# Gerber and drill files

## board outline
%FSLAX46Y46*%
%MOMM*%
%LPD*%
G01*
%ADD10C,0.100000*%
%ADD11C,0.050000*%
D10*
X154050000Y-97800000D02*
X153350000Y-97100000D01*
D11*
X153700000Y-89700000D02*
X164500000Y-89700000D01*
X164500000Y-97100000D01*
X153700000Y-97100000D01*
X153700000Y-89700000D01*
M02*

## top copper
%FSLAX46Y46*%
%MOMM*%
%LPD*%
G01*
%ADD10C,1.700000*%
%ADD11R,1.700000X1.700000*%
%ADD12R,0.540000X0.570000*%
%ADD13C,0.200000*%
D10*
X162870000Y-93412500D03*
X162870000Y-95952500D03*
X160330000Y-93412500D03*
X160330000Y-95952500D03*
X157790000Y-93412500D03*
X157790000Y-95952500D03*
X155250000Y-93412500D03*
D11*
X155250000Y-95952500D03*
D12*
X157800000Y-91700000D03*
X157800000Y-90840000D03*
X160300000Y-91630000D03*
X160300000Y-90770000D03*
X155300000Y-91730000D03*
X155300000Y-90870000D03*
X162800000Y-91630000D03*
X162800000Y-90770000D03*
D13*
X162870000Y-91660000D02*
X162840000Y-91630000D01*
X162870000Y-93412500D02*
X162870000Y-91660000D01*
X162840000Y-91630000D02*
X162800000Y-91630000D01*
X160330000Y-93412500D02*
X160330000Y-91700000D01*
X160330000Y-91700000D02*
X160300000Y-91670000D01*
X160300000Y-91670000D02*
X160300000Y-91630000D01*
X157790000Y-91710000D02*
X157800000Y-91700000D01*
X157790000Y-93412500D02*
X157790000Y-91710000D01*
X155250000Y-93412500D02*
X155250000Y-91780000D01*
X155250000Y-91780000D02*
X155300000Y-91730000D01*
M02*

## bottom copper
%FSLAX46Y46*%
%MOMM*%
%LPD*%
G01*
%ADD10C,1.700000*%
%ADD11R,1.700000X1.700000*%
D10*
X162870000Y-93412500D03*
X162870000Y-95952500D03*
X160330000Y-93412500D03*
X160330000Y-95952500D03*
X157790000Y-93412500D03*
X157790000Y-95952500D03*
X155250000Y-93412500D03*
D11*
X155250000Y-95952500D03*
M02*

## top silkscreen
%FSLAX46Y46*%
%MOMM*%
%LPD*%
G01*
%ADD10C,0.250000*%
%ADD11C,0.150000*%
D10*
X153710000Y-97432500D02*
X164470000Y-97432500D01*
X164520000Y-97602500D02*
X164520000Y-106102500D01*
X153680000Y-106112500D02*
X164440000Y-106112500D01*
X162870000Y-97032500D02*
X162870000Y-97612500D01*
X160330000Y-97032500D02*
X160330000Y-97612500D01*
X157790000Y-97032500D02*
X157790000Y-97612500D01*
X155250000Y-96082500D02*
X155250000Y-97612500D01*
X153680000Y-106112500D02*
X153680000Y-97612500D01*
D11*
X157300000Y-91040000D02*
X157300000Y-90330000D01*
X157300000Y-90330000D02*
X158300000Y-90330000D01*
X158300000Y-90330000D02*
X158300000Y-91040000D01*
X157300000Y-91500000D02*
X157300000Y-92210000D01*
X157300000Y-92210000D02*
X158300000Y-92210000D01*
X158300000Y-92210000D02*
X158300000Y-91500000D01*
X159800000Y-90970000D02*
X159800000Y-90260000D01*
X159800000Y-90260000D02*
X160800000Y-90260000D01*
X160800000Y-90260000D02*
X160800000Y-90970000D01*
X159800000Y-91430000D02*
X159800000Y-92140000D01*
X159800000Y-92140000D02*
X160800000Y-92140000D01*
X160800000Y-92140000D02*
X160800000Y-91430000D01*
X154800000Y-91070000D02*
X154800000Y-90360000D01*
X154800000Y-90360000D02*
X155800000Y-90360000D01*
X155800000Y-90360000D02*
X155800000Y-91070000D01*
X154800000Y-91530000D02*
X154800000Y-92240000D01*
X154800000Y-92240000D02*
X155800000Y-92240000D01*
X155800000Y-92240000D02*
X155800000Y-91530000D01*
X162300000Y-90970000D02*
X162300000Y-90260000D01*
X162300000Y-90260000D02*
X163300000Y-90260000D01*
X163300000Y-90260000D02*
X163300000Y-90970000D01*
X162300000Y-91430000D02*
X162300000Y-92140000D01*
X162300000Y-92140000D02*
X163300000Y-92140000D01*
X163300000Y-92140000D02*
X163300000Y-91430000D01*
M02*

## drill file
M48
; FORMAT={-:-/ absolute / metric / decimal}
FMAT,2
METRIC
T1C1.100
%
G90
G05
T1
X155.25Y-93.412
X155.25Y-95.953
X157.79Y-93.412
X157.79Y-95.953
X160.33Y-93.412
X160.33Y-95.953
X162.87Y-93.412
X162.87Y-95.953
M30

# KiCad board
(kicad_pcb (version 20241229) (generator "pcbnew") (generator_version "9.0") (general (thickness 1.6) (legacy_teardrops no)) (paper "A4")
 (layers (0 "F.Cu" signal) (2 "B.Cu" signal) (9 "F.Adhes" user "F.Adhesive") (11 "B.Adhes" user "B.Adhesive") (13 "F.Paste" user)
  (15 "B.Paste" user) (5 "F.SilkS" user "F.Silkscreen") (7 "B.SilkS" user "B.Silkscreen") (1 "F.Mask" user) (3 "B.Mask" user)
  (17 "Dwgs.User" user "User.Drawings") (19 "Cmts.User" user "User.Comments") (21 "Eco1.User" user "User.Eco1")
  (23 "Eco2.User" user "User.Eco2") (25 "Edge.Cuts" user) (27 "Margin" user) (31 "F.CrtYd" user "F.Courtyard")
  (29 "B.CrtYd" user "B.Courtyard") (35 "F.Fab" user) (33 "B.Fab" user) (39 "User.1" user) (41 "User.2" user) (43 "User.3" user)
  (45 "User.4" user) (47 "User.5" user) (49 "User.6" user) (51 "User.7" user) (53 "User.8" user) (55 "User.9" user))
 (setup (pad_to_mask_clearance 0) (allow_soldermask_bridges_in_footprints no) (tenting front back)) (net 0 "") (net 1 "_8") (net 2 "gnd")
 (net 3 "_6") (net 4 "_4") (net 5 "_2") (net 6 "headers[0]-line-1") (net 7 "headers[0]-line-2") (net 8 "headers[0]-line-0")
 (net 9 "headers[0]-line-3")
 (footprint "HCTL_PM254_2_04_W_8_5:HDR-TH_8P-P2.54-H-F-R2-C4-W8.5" (layer "F.Cu") (at 159.06 94.6825 0)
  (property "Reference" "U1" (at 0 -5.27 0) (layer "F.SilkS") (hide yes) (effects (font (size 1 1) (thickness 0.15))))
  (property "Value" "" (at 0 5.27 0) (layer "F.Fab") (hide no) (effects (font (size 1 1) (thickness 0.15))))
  (fp_line (start -5.35 2.75) (end 5.41 2.75) (stroke (width 0.25) (type solid)) (layer "F.SilkS"))
  (fp_line (start 5.46 2.92) (end 5.46 11.42) (stroke (width 0.25) (type solid)) (layer "F.SilkS"))
  (fp_line (start -5.38 11.43) (end 5.38 11.43) (stroke (width 0.25) (type solid)) (layer "F.SilkS"))
  (fp_line (start 3.81 2.35) (end 3.81 2.93) (stroke (width 0.25) (type solid)) (layer "F.SilkS"))
  (fp_line (start 1.27 2.35) (end 1.27 2.93) (stroke (width 0.25) (type solid)) (layer "F.SilkS"))
  (fp_line (start -1.27 2.35) (end -1.27 2.93) (stroke (width 0.25) (type solid)) (layer "F.SilkS"))
  (fp_line (start -3.81 1.4) (end -3.81 2.93) (stroke (width 0.25) (type solid)) (layer "F.SilkS"))
  (fp_line (start -5.38 11.43) (end -5.38 2.93) (stroke (width 0.25) (type solid)) (layer "F.SilkS"))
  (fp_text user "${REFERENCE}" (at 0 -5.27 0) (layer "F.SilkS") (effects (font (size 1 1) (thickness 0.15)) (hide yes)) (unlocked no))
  (pad "8" thru_hole circle (at 3.81 -1.27 0) (size 1.7 1.7) (drill 1.1000231999999999) (layers "*.Cu" "*.Mask") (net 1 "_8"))
  (pad "7" thru_hole circle (at 3.81 1.27 0) (size 1.7 1.7) (drill 1.1000231999999999) (layers "*.Cu" "*.Mask") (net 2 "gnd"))
  (pad "6" thru_hole circle (at 1.27 -1.27 0) (size 1.7 1.7) (drill 1.1000231999999999) (layers "*.Cu" "*.Mask") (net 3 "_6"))
  (pad "5" thru_hole circle (at 1.27 1.27 0) (size 1.7 1.7) (drill 1.1000231999999999) (layers "*.Cu" "*.Mask") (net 2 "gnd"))
  (pad "4" thru_hole circle (at -1.27 -1.27 0) (size 1.7 1.7) (drill 1.1000231999999999) (layers "*.Cu" "*.Mask") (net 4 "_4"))
  (pad "3" thru_hole circle (at -1.27 1.27 0) (size 1.7 1.7) (drill 1.1000231999999999) (layers "*.Cu" "*.Mask") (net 2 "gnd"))
  (pad "2" thru_hole circle (at -3.81 -1.27 0) (size 1.7 1.7) (drill 1.1000231999999999) (layers "*.Cu" "*.Mask") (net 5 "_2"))
  (pad "1" thru_hole rect (at -3.81 1.27 0) (size 1.7 1.7) (drill 1.1000231999999999) (layers "*.Cu" "*.Mask") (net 2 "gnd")))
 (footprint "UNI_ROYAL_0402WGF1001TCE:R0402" (layer "F.Cu") (at 157.8 91.27 -90)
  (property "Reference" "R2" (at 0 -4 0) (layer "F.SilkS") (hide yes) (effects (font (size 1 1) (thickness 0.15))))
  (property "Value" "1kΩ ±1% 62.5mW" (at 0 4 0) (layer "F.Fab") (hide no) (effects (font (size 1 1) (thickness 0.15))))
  (fp_line (start -0.23 0.5) (end -0.94 0.5) (stroke (width 0.15) (type solid)) (layer "F.SilkS"))
  (fp_line (start -0.94 0.5) (end -0.94 -0.5) (stroke (width 0.15) (type solid)) (layer "F.SilkS"))
  (fp_line (start -0.94 -0.5) (end -0.23 -0.5) (stroke (width 0.15) (type solid)) (layer "F.SilkS"))
  (fp_line (start 0.23 0.5) (end 0.94 0.5) (stroke (width 0.15) (type solid)) (layer "F.SilkS"))
  (fp_line (start 0.94 0.5) (end 0.94 -0.5) (stroke (width 0.15) (type solid)) (layer "F.SilkS"))
  (fp_line (start 0.94 -0.5) (end 0.23 -0.5) (stroke (width 0.15) (type solid)) (layer "F.SilkS"))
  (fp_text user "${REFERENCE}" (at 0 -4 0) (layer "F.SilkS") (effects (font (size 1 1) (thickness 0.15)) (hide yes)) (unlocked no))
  (pad "2" smd rect (at 0.43 0 -90) (size 0.57 0.54) (layers "F.Cu" "F.Paste" "F.Mask") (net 4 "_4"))
  (pad "1" smd rect (at -0.43 0 -90) (size 0.57 0.54) (layers "F.Cu" "F.Paste" "F.Mask") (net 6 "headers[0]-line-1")))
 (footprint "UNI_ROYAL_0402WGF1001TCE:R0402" (layer "F.Cu") (at 160.3 91.2 -90)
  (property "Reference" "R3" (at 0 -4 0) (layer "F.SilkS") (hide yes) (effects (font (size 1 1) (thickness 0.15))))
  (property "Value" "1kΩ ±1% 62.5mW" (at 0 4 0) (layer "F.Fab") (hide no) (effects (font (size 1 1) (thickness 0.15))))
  (fp_line (start -0.23 0.5) (end -0.94 0.5) (stroke (width 0.15) (type solid)) (layer "F.SilkS"))
  (fp_line (start -0.94 0.5) (end -0.94 -0.5) (stroke (width 0.15) (type solid)) (layer "F.SilkS"))
  (fp_line (start -0.94 -0.5) (end -0.23 -0.5) (stroke (width 0.15) (type solid)) (layer "F.SilkS"))
  (fp_line (start 0.23 0.5) (end 0.94 0.5) (stroke (width 0.15) (type solid)) (layer "F.SilkS"))
  (fp_line (start 0.94 0.5) (end 0.94 -0.5) (stroke (width 0.15) (type solid)) (layer "F.SilkS"))
  (fp_line (start 0.94 -0.5) (end 0.23 -0.5) (stroke (width 0.15) (type solid)) (layer "F.SilkS"))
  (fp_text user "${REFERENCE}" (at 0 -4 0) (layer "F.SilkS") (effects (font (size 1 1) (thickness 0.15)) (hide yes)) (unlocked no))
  (pad "2" smd rect (at 0.43 0 -90) (size 0.57 0.54) (layers "F.Cu" "F.Paste" "F.Mask") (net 3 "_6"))
  (pad "1" smd rect (at -0.43 0 -90) (size 0.57 0.54) (layers "F.Cu" "F.Paste" "F.Mask") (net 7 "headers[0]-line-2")))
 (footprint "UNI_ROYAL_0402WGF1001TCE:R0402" (layer "F.Cu") (at 155.3 91.3 -90)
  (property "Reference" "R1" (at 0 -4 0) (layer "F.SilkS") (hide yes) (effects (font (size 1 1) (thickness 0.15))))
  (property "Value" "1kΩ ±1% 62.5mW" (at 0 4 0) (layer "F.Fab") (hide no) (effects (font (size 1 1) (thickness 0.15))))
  (fp_line (start -0.23 0.5) (end -0.94 0.5) (stroke (width 0.15) (type solid)) (layer "F.SilkS"))
  (fp_line (start -0.94 0.5) (end -0.94 -0.5) (stroke (width 0.15) (type solid)) (layer "F.SilkS"))
  (fp_line (start -0.94 -0.5) (end -0.23 -0.5) (stroke (width 0.15) (type solid)) (layer "F.SilkS"))
  (fp_line (start 0.23 0.5) (end 0.94 0.5) (stroke (width 0.15) (type solid)) (layer "F.SilkS"))
  (fp_line (start 0.94 0.5) (end 0.94 -0.5) (stroke (width 0.15) (type solid)) (layer "F.SilkS"))
  (fp_line (start 0.94 -0.5) (end 0.23 -0.5) (stroke (width 0.15) (type solid)) (layer "F.SilkS"))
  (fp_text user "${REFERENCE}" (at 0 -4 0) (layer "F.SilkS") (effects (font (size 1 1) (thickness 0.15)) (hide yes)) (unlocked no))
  (pad "2" smd rect (at 0.43 0 -90) (size 0.57 0.54) (layers "F.Cu" "F.Paste" "F.Mask") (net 5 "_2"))
  (pad "1" smd rect (at -0.43 0 -90) (size 0.57 0.54) (layers "F.Cu" "F.Paste" "F.Mask") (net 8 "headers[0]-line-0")))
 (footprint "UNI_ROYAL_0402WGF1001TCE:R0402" (layer "F.Cu") (at 162.8 91.2 -90)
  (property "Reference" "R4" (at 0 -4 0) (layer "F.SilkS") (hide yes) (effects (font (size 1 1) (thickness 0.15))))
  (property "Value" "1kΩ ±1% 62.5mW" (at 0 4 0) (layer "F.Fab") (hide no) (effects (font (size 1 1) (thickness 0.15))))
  (fp_line (start -0.23 0.5) (end -0.94 0.5) (stroke (width 0.15) (type solid)) (layer "F.SilkS"))
  (fp_line (start -0.94 0.5) (end -0.94 -0.5) (stroke (width 0.15) (type solid)) (layer "F.SilkS"))
  (fp_line (start -0.94 -0.5) (end -0.23 -0.5) (stroke (width 0.15) (type solid)) (layer "F.SilkS"))
  (fp_line (start 0.23 0.5) (end 0.94 0.5) (stroke (width 0.15) (type solid)) (layer "F.SilkS"))
  (fp_line (start 0.94 0.5) (end 0.94 -0.5) (stroke (width 0.15) (type solid)) (layer "F.SilkS"))
  (fp_line (start 0.94 -0.5) (end 0.23 -0.5) (stroke (width 0.15) (type solid)) (layer "F.SilkS"))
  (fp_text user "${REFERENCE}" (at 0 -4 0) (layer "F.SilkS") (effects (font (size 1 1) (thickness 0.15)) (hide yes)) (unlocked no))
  (pad "2" smd rect (at 0.43 0 -90) (size 0.57 0.54) (layers "F.Cu" "F.Paste" "F.Mask") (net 1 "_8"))
  (pad "1" smd rect (at -0.43 0 -90) (size 0.57 0.54) (layers "F.Cu" "F.Paste" "F.Mask") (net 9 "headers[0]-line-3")))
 (segment (start 162.87 91.66) (end 162.84 91.63) (width 0.2) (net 1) (layer "F.Cu"))
 (segment (start 162.87 93.4125) (end 162.87 91.66) (width 0.2) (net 1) (layer "F.Cu"))
 (segment (start 162.84 91.63) (end 162.8 91.63) (width 0.2) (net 1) (layer "F.Cu"))
 (segment (start 160.33 93.4125) (end 160.33 91.7) (width 0.2) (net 3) (layer "F.Cu"))
 (segment (start 160.33 91.7) (end 160.3 91.67) (width 0.2) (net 3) (layer "F.Cu"))
 (segment (start 160.3 91.67) (end 160.3 91.63) (width 0.2) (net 3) (layer "F.Cu"))
 (segment (start 157.79 91.71) (end 157.8 91.7) (width 0.2) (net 4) (layer "F.Cu"))
 (segment (start 157.79 93.4125) (end 157.79 91.71) (width 0.2) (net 4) (layer "F.Cu"))
 (segment (start 155.25 93.4125) (end 155.25 91.78) (width 0.2) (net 5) (layer "F.Cu"))
 (segment (start 155.25 91.78) (end 155.3 91.73) (width 0.2) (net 5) (layer "F.Cu"))
 (gr_line (start 154.05 97.8) (end 153.35 97.1) (stroke (width 0.1) (type solid)) (layer "Edge.Cuts"))
 (gr_rect (start 153.7 89.7) (end 164.5 97.1) (stroke (width 0.05) (type default)) (fill no) (layer "Edge.Cuts")))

